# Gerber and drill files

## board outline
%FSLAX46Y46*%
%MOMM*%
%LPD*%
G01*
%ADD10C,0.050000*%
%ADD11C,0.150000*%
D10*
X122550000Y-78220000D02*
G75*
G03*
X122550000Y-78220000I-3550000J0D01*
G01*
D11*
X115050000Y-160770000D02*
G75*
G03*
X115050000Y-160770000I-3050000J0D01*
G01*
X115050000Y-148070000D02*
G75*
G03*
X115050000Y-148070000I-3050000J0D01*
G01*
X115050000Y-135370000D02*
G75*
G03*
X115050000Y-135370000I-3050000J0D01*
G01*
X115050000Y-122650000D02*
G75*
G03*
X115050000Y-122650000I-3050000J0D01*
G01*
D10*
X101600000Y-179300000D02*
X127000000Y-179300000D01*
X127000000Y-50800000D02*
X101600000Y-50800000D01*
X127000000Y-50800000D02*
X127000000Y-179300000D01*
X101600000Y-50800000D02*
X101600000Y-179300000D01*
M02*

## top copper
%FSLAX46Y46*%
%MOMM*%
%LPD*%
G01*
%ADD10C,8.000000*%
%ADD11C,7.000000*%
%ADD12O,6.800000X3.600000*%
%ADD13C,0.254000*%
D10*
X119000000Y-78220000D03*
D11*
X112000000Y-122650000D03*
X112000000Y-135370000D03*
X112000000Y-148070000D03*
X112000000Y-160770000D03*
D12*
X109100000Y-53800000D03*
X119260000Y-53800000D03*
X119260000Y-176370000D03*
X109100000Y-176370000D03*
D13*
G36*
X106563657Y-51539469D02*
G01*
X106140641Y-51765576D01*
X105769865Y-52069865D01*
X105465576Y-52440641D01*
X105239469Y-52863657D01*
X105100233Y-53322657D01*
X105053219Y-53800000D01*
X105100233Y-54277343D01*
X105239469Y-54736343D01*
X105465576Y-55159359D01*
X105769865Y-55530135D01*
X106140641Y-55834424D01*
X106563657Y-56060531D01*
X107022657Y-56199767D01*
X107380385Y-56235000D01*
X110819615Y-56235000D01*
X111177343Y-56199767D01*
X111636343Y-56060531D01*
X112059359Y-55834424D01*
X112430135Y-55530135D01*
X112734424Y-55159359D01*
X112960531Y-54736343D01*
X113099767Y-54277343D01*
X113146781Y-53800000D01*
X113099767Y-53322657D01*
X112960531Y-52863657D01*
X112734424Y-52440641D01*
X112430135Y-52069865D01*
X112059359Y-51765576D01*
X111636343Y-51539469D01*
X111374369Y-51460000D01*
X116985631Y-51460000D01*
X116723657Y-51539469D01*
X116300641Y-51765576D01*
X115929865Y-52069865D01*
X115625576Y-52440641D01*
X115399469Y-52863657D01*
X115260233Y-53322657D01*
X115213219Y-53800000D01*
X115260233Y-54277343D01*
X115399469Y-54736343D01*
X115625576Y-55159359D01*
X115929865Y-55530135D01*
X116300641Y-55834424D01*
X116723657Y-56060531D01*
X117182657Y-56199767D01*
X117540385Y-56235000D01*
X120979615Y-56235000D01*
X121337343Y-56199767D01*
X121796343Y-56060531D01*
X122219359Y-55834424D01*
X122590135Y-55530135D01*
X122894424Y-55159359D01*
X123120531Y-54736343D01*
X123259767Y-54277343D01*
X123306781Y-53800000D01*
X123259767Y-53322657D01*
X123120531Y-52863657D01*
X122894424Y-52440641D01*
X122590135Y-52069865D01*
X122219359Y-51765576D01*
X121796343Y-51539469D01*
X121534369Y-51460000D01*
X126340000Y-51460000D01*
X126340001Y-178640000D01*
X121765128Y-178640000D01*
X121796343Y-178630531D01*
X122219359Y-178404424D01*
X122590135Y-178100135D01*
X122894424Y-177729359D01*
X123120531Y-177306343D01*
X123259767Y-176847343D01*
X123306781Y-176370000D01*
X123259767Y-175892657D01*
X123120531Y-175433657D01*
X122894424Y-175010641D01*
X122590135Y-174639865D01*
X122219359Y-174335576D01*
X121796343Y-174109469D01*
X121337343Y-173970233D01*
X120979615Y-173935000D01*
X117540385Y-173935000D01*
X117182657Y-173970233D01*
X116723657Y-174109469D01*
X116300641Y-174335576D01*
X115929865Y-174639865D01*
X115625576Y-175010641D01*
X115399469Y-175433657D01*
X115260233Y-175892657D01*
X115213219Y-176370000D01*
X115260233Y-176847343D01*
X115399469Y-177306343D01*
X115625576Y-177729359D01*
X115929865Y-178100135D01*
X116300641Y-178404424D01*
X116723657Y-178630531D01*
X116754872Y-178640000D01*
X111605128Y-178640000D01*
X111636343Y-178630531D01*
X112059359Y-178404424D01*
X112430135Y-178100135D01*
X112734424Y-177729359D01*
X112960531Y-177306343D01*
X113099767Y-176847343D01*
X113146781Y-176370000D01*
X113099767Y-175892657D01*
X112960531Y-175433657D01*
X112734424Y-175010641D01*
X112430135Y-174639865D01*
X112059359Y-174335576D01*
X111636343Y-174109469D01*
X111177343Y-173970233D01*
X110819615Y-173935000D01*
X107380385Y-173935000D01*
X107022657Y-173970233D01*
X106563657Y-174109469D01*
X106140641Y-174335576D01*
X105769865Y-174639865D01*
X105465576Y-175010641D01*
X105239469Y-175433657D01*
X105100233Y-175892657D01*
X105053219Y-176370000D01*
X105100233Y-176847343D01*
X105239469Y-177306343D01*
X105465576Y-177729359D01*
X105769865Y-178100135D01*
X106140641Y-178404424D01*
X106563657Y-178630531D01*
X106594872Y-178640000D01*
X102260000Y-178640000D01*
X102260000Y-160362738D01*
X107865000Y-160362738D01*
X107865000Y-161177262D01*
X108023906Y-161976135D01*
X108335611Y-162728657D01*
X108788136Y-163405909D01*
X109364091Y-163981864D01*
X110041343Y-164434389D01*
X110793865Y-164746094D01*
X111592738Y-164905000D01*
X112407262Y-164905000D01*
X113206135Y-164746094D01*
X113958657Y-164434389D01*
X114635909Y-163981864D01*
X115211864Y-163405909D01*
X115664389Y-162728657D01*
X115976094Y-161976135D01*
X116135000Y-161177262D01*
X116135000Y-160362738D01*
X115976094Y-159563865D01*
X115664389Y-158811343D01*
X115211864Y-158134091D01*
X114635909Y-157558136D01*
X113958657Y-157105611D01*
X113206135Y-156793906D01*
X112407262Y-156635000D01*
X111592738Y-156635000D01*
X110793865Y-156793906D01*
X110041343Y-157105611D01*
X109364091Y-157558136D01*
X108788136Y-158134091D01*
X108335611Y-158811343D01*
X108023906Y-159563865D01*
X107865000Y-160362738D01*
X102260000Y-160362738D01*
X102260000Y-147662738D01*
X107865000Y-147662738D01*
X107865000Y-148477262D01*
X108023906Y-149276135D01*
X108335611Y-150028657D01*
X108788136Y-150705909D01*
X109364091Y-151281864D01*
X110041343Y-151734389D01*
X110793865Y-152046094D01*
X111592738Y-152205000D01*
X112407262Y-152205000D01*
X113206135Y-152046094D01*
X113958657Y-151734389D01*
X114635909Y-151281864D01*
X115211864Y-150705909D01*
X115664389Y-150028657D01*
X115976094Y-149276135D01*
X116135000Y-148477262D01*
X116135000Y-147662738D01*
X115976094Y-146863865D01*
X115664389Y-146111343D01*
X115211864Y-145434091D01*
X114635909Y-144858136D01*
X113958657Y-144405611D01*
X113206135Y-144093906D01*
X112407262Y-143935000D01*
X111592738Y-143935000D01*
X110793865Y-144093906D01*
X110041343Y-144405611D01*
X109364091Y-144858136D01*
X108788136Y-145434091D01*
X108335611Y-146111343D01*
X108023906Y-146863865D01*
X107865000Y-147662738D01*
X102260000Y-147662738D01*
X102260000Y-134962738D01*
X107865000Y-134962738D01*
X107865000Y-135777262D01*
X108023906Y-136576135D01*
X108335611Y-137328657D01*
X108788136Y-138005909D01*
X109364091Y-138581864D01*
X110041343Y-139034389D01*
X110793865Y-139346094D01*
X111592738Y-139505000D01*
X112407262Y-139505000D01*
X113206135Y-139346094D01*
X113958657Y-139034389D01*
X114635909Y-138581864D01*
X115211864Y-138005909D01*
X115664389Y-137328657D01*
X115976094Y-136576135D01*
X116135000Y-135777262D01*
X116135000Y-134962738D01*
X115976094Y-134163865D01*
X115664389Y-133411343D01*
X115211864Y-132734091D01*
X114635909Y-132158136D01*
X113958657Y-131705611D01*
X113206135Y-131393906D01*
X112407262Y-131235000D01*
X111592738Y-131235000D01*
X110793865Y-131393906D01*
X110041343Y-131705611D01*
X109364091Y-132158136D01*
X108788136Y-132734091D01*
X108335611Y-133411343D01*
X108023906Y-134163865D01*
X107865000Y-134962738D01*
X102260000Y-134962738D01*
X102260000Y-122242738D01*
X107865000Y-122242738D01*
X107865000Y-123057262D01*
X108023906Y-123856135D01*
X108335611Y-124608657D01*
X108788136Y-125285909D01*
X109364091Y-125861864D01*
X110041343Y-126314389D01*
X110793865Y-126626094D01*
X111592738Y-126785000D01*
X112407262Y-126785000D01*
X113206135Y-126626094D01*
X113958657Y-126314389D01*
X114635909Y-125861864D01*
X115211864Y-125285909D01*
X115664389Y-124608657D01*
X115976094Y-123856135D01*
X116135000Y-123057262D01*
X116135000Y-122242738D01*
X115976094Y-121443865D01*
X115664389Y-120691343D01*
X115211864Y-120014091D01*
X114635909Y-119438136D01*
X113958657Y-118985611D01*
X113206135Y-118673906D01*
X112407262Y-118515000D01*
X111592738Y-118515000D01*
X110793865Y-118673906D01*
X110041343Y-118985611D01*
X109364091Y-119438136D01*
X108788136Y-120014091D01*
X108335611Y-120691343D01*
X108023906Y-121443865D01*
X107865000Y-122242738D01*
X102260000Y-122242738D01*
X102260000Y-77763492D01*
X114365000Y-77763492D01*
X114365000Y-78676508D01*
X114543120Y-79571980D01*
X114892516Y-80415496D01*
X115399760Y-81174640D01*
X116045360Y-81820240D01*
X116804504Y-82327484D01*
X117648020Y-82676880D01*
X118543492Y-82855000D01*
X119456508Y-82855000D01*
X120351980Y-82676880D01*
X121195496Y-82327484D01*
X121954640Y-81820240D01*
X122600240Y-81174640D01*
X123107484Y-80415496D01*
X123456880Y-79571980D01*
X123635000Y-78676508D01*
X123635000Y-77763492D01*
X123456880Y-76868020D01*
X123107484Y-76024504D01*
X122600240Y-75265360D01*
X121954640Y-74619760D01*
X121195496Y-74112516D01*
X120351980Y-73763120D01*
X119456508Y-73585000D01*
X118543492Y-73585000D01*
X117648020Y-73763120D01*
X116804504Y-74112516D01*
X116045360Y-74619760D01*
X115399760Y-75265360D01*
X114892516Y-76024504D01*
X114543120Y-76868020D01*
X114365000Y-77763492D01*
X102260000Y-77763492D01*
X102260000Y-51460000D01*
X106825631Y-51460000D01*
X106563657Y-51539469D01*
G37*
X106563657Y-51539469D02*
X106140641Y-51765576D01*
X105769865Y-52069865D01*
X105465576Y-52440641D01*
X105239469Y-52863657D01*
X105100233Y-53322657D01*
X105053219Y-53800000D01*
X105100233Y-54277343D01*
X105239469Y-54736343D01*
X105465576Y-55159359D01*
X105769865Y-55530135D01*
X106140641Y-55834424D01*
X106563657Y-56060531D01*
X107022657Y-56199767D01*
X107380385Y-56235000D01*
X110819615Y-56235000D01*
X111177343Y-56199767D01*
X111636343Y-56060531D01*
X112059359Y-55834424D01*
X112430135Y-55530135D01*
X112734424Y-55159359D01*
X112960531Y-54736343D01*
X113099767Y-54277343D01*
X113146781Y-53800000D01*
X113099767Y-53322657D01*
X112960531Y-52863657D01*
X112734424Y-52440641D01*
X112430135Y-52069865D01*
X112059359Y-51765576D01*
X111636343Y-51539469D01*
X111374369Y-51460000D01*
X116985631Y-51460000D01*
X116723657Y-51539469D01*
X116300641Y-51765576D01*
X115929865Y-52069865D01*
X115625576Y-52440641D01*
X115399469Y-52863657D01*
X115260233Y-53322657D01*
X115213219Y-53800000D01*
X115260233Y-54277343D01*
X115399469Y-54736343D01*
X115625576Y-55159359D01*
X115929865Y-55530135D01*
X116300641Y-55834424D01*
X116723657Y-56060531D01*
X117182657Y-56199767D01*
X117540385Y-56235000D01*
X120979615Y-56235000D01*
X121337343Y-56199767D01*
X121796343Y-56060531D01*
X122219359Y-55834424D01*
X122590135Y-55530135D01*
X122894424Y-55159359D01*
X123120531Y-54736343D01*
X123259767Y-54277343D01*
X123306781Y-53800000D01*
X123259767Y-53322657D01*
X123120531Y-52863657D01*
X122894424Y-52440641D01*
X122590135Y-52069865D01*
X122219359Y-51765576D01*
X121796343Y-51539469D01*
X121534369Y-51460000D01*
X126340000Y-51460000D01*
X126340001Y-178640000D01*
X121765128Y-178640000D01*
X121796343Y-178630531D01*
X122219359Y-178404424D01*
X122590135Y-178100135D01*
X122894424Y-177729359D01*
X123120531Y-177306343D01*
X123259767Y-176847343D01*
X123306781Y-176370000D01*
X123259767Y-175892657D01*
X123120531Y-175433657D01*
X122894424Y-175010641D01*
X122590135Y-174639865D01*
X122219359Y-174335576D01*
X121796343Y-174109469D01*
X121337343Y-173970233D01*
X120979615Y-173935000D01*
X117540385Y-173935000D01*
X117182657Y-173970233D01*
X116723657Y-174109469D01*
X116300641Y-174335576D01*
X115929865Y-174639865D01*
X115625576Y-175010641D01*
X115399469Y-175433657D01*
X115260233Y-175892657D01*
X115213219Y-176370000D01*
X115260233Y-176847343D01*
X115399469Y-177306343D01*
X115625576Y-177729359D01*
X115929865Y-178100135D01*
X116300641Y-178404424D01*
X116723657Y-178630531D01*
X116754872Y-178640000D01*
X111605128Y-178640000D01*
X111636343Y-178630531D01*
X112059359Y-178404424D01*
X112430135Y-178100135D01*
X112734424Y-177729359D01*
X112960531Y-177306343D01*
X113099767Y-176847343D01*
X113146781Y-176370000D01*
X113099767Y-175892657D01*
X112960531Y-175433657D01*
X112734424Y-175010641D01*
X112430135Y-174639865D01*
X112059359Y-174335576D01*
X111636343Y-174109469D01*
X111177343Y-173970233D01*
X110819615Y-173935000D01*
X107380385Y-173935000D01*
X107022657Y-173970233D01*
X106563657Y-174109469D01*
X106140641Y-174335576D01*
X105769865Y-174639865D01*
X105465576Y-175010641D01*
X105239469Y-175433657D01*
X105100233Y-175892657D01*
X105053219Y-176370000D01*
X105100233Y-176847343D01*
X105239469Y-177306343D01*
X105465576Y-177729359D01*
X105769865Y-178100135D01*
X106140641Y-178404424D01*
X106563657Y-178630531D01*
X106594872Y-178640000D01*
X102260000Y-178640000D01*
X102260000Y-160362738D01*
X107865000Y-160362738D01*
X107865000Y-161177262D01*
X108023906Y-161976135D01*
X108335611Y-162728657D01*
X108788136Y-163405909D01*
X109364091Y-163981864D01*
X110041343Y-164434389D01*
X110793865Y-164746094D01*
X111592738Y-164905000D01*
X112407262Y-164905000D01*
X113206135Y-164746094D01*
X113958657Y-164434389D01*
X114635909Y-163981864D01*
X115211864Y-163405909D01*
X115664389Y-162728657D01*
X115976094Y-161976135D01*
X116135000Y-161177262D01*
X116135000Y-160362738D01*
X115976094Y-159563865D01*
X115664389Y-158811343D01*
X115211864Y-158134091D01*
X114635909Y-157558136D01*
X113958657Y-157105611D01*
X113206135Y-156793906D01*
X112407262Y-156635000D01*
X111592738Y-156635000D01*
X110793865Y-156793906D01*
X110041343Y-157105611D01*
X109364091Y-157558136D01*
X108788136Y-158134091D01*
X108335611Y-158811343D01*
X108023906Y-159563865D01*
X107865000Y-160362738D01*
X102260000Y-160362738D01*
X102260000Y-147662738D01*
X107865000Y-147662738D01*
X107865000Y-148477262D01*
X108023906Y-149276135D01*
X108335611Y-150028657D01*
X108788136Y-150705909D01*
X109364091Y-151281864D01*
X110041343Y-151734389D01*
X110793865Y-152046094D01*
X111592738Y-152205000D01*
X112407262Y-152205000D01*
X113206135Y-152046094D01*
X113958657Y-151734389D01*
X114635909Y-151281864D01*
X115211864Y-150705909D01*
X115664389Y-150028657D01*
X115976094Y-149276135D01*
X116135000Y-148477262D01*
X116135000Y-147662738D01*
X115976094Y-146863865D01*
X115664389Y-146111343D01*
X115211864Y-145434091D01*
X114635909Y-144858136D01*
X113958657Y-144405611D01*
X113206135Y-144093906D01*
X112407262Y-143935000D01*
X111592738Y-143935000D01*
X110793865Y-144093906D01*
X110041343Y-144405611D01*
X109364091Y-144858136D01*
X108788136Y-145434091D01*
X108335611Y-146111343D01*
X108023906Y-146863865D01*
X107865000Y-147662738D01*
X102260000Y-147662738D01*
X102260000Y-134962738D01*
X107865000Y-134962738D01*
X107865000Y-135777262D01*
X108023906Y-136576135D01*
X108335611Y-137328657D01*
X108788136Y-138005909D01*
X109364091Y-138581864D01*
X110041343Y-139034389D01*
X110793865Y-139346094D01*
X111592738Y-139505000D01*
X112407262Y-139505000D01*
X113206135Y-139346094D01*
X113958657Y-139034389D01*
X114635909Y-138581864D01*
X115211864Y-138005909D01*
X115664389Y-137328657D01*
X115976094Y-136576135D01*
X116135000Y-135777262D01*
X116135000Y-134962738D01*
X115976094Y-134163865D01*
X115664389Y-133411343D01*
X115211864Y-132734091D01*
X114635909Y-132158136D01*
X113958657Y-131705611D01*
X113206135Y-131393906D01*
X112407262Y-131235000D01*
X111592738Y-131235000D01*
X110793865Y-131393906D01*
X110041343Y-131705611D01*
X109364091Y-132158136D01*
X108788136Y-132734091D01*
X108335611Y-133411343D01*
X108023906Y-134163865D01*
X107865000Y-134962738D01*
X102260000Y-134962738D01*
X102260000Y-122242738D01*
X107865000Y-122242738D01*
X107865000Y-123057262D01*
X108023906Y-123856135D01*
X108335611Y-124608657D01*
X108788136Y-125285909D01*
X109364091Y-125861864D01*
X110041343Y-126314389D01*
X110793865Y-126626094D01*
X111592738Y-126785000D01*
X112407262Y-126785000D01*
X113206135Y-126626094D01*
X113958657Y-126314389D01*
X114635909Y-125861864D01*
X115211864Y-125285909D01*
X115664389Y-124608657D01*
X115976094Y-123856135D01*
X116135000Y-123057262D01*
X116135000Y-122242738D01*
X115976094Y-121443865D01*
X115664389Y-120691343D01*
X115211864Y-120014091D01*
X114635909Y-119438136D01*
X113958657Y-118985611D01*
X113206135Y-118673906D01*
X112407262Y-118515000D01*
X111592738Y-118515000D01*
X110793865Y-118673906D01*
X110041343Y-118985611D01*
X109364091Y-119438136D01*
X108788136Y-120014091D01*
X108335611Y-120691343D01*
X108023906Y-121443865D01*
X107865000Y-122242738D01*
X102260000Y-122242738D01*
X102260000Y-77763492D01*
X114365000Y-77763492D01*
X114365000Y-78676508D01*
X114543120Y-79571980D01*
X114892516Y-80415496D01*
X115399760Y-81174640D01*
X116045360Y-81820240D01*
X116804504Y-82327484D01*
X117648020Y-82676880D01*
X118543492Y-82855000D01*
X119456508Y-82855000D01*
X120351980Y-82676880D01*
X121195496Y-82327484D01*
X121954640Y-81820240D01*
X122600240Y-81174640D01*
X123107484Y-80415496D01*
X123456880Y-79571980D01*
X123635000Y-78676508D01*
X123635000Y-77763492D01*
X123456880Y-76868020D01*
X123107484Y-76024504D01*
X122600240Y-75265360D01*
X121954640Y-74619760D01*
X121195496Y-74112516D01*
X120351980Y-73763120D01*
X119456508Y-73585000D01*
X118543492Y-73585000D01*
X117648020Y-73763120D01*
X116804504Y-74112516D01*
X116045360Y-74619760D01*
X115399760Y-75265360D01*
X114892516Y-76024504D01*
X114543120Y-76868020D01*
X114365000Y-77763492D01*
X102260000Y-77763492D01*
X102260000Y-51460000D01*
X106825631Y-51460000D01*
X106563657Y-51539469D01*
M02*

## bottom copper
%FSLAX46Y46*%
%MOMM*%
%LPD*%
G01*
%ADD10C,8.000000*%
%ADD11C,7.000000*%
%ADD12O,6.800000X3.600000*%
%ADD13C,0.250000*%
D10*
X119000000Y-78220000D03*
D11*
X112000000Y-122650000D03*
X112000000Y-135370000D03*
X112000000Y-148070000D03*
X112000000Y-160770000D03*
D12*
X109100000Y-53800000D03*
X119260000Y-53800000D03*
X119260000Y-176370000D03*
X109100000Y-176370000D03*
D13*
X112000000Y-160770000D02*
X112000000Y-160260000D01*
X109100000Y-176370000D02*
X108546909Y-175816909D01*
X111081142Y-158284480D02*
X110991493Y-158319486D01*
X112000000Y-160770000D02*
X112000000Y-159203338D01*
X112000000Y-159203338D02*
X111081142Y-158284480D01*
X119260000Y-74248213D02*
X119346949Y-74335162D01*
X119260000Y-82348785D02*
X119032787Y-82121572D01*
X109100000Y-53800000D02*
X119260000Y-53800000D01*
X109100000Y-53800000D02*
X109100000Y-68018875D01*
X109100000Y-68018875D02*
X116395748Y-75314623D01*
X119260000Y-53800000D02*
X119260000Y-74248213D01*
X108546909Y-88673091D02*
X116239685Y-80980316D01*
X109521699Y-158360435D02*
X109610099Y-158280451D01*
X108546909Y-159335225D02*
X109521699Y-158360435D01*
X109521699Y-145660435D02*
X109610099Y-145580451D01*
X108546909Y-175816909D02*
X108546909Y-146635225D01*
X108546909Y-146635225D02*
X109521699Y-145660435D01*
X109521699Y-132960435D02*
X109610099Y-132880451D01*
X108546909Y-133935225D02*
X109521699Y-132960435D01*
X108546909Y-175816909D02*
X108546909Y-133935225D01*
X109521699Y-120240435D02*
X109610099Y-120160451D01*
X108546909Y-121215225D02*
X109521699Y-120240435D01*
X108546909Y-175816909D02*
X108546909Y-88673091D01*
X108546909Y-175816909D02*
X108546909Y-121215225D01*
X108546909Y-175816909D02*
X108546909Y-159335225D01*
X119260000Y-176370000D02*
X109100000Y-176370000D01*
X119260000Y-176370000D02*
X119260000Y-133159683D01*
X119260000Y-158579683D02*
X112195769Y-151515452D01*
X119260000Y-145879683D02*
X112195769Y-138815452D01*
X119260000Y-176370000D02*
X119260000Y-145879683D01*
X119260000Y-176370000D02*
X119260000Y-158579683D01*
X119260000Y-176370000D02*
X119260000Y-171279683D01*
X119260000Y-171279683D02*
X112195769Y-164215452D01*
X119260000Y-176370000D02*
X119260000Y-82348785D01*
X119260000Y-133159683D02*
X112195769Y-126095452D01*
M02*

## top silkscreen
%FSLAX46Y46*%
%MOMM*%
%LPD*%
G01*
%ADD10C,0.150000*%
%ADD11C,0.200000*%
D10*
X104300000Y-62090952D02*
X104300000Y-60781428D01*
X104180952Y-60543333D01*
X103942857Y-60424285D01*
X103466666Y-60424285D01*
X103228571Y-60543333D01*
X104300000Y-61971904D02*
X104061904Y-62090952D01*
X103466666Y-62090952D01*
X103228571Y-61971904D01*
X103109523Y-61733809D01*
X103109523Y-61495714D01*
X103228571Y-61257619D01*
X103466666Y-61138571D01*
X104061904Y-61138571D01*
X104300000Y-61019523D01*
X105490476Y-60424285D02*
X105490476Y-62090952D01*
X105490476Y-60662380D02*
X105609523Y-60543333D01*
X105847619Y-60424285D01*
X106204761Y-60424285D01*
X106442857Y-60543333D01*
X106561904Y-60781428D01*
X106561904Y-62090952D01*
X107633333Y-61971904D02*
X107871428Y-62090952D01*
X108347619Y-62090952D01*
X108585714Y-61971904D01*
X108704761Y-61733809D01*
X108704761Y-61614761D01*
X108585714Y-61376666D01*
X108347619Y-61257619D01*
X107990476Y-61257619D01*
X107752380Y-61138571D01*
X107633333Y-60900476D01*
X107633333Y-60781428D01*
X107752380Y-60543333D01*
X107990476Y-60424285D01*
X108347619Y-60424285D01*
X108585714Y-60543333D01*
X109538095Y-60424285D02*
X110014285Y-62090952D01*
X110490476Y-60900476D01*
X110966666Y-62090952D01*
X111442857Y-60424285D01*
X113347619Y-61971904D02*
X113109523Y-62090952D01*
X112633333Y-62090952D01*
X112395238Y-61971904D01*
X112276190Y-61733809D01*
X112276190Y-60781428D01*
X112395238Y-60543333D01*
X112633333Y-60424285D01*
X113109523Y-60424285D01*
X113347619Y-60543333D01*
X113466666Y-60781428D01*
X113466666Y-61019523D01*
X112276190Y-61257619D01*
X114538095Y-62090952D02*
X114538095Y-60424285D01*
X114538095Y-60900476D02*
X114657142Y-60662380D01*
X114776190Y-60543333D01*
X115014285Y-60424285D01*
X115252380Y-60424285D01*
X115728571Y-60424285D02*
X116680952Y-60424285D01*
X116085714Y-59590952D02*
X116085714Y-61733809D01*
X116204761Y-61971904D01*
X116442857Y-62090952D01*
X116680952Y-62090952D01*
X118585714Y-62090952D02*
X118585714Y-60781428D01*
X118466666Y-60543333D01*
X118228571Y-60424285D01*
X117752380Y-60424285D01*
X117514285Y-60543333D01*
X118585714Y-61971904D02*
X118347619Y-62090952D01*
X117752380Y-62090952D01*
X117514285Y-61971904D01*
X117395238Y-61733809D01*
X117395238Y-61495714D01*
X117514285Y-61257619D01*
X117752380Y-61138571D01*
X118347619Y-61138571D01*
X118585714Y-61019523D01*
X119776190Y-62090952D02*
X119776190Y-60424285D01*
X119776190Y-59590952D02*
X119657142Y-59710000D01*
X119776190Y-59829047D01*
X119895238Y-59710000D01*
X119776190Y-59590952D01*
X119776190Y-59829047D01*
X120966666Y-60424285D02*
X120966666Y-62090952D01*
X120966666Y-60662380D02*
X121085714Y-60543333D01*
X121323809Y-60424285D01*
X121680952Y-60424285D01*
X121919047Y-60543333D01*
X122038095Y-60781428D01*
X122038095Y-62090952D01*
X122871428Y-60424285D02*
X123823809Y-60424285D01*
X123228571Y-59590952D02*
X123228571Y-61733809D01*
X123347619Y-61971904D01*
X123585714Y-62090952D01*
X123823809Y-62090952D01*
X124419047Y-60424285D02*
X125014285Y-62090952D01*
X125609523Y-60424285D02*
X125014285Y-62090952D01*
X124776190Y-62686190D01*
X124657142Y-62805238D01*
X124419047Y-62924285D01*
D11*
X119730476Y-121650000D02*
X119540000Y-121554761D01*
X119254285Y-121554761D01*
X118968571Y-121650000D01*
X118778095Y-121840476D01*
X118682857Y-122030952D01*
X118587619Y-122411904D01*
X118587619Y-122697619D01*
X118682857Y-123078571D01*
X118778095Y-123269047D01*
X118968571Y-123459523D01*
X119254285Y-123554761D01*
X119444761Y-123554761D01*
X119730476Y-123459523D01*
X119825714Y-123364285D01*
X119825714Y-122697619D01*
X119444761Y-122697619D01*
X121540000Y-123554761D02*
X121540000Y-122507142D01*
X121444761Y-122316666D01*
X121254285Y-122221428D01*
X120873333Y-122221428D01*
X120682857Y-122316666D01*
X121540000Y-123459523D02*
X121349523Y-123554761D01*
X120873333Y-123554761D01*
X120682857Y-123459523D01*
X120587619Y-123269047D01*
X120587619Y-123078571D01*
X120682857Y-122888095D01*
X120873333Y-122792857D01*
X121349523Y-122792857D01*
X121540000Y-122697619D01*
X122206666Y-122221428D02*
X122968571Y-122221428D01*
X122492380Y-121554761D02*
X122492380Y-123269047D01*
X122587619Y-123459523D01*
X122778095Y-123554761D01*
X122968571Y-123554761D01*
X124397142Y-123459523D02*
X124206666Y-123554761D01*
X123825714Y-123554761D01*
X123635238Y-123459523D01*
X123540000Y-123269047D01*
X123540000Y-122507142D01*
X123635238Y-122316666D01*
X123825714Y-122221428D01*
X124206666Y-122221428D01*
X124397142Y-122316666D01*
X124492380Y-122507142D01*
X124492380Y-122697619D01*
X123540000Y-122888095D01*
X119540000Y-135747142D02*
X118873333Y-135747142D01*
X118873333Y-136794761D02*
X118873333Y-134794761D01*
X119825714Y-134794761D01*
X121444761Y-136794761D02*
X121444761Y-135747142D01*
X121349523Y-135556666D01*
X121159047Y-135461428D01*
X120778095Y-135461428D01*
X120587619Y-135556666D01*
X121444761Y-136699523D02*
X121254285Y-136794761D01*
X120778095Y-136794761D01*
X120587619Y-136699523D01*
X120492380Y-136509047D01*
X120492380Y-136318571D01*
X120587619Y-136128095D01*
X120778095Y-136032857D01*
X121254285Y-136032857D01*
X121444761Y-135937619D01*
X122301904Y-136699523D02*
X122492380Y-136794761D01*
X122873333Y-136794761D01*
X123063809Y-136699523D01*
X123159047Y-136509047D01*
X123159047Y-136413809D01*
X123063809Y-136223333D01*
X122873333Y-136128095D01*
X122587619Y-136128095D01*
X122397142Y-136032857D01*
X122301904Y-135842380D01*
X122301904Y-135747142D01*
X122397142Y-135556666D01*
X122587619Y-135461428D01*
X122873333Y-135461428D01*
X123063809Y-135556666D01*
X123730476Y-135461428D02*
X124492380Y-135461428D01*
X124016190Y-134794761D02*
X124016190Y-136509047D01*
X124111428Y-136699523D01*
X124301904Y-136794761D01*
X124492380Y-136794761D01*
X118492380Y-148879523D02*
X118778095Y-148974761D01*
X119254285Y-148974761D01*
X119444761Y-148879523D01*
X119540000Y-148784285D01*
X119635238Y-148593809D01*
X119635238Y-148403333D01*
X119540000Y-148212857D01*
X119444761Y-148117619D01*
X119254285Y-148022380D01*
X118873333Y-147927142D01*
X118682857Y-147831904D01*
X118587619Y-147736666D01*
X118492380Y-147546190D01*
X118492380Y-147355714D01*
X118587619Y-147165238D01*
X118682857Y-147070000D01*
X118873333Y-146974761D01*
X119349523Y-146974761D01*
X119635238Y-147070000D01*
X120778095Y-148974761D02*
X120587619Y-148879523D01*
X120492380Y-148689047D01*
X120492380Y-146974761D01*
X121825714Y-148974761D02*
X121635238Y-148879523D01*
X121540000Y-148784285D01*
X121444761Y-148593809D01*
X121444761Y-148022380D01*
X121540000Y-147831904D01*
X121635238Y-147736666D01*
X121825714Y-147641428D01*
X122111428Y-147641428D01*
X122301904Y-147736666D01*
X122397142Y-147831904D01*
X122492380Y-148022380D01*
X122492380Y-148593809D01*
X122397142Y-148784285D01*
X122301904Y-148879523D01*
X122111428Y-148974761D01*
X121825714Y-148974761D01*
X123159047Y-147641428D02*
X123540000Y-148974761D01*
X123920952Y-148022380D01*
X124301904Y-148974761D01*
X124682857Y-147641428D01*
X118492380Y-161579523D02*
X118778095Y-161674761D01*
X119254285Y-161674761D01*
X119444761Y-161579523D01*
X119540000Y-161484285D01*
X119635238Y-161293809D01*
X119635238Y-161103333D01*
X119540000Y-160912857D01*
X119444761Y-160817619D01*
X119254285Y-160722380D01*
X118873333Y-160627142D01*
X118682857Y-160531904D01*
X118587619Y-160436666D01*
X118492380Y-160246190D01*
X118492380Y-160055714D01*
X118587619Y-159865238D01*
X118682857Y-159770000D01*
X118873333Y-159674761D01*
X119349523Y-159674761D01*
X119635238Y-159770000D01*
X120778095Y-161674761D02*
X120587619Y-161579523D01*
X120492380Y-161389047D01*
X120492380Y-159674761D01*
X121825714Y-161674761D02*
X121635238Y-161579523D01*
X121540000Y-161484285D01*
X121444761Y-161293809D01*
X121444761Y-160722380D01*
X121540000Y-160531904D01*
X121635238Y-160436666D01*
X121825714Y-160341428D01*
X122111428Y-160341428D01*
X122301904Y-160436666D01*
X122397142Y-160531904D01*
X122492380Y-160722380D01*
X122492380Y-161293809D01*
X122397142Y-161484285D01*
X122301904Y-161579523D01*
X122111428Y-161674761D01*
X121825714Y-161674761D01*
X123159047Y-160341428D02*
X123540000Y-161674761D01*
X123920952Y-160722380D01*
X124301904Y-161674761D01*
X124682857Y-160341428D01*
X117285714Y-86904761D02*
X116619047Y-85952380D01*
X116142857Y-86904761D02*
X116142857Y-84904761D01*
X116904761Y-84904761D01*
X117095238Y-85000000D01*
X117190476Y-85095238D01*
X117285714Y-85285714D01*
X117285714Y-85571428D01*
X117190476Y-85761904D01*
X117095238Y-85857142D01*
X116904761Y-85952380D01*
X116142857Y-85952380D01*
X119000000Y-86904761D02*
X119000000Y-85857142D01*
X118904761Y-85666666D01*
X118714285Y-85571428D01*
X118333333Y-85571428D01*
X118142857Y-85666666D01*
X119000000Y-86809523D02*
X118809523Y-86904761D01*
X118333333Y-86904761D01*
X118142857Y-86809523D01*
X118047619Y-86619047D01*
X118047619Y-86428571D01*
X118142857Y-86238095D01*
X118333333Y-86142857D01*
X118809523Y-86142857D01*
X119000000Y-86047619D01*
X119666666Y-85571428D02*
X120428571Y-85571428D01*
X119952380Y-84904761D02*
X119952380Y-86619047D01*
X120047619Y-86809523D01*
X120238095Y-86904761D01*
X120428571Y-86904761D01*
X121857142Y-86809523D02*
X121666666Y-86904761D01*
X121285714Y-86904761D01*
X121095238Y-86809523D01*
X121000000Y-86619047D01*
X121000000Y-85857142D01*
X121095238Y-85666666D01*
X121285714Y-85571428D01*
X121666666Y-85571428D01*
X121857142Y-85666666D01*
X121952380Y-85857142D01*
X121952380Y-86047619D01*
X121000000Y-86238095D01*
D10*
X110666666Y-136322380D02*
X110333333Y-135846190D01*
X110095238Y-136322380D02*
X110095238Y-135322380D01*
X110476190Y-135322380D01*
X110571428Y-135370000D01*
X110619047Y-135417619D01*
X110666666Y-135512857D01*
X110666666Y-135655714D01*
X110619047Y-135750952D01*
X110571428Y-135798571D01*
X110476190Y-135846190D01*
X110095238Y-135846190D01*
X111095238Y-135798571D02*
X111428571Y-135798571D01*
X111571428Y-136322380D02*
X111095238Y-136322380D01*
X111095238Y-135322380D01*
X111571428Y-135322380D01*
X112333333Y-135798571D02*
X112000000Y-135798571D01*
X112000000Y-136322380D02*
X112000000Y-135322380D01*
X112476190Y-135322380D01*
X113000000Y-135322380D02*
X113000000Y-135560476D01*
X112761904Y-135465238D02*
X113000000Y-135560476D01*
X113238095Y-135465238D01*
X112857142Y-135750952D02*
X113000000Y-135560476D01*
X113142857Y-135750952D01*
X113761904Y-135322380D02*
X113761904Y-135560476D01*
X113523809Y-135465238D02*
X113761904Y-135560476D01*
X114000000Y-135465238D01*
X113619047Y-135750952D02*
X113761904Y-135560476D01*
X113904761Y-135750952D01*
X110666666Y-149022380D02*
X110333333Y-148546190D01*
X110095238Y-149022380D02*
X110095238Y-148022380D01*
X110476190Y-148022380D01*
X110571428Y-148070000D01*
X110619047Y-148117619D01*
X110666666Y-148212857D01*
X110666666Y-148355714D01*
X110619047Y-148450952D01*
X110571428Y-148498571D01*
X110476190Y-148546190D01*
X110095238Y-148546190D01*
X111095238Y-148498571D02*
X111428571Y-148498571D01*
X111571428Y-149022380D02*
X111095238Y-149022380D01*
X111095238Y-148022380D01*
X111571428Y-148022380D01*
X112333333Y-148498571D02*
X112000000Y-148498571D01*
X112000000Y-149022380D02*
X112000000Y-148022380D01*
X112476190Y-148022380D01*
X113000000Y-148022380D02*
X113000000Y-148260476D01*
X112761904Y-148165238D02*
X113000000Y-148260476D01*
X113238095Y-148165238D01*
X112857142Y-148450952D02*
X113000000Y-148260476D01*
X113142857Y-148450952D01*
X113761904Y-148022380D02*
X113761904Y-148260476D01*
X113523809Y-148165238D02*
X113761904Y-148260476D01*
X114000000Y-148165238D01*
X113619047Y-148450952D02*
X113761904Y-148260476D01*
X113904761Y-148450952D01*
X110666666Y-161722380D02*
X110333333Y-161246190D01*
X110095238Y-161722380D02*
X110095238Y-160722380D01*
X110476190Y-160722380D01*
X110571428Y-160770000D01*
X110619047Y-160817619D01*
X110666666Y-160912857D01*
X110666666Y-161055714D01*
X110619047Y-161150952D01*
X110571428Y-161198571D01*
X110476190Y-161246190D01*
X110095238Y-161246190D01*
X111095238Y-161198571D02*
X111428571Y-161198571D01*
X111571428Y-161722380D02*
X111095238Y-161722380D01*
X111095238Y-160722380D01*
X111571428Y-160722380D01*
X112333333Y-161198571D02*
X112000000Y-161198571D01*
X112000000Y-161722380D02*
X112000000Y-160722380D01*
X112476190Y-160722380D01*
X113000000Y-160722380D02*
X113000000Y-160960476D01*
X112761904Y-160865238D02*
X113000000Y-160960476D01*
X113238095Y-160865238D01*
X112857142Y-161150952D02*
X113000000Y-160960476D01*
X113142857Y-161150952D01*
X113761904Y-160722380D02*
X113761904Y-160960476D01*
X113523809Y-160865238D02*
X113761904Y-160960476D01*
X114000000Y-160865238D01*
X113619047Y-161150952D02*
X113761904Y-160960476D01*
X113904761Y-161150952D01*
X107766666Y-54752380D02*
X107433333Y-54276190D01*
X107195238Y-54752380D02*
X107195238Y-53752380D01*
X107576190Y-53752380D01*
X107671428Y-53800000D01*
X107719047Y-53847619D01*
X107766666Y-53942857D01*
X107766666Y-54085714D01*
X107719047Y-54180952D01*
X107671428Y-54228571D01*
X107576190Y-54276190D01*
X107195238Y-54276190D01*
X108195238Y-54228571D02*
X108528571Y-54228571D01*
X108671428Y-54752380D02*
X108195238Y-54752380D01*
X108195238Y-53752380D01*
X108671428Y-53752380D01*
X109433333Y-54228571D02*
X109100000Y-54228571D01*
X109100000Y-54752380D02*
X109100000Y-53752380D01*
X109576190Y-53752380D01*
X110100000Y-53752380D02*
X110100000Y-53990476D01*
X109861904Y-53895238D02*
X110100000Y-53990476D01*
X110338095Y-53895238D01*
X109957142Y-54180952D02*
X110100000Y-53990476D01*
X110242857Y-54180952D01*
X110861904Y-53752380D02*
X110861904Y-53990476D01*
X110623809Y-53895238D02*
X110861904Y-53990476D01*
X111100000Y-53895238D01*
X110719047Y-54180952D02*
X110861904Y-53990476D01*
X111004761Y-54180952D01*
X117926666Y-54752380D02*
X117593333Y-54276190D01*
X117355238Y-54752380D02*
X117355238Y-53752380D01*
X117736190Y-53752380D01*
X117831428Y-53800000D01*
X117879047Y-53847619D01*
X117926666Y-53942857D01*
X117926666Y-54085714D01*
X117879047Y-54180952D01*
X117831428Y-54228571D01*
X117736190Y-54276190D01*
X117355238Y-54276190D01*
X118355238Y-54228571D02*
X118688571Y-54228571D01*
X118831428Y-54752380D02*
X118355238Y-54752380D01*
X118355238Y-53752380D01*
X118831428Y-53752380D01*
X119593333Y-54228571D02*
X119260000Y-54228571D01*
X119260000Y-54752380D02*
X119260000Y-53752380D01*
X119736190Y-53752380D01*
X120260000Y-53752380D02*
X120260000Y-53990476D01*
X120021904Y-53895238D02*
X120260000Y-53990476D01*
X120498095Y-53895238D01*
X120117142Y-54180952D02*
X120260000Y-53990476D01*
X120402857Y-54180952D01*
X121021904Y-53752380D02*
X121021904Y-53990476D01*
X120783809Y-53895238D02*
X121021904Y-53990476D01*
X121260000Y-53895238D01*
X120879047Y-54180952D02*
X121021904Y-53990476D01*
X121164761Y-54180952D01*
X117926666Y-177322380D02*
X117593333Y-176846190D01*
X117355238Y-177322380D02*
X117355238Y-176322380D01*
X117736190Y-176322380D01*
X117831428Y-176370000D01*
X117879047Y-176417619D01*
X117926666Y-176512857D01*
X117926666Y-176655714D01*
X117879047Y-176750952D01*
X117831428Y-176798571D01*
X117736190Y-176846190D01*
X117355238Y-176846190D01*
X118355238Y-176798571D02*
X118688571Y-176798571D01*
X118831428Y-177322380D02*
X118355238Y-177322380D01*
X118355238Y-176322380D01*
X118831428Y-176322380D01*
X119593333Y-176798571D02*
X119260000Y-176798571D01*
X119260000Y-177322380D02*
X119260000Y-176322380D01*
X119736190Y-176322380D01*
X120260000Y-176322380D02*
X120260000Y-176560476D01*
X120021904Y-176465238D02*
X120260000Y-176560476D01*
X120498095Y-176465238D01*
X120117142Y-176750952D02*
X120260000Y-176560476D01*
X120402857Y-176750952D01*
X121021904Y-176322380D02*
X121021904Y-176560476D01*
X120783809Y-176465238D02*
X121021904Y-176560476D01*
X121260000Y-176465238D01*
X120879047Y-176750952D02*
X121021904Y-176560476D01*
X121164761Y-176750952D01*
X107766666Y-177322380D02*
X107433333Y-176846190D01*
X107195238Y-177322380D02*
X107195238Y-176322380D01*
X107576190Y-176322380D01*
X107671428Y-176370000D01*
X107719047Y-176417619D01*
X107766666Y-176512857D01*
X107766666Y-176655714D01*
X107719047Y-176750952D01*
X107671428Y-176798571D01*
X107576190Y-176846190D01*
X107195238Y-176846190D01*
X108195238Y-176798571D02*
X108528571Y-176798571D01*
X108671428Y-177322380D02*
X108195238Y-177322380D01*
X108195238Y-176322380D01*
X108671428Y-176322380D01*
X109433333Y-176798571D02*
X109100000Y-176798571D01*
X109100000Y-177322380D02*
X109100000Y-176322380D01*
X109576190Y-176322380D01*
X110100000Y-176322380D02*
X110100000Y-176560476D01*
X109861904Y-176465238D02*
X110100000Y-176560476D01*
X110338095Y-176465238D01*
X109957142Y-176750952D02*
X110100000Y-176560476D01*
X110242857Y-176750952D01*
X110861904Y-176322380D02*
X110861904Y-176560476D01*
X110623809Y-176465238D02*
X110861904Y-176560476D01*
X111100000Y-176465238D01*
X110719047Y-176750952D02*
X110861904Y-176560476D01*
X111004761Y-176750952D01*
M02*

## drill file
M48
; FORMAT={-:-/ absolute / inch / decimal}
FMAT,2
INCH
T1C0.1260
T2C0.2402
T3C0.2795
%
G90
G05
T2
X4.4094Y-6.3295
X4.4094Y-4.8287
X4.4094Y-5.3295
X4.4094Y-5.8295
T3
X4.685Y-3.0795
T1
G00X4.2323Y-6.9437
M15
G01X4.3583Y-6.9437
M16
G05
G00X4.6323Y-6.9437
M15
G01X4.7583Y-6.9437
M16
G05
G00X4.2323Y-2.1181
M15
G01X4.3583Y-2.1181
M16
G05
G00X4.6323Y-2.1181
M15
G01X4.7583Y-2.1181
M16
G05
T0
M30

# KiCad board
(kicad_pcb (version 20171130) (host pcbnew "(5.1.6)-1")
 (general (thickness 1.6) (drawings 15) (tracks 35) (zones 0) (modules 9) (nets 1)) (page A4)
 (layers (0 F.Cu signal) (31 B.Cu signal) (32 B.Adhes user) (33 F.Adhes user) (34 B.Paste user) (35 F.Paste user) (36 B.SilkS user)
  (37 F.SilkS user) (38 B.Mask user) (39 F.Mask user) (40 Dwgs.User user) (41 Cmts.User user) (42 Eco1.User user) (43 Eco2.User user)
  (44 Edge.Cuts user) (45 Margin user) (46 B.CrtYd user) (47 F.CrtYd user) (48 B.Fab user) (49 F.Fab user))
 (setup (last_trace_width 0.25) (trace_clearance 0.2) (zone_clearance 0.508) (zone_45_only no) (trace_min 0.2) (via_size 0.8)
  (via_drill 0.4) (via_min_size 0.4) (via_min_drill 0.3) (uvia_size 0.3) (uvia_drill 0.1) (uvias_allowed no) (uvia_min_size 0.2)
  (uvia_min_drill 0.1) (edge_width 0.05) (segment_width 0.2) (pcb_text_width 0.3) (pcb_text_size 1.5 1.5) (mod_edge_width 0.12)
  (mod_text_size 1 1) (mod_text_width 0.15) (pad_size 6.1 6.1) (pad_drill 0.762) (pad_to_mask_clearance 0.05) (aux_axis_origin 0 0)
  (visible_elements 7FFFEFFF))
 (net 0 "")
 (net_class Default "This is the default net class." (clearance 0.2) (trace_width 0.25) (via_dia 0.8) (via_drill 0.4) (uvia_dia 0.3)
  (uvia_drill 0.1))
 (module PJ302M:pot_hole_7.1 (layer F.Cu) (at 119 78.22)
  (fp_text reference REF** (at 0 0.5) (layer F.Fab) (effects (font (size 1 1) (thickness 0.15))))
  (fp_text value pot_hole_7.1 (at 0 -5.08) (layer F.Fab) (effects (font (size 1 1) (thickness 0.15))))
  (pad "" np_thru_hole circle (at 0 0) (size 8 8) (drill 7.1) (layers *.Cu *.Mask)))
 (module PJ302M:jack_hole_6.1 (layer F.Cu) (at 112 122.65)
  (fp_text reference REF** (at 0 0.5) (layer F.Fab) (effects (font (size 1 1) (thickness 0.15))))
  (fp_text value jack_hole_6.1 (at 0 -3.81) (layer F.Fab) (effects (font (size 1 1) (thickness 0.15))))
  (pad "" np_thru_hole circle (at 0 0 90) (size 7 7) (drill 6.1) (layers *.Cu *.Mask)))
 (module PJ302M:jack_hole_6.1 (layer F.Cu) (at 112 135.37)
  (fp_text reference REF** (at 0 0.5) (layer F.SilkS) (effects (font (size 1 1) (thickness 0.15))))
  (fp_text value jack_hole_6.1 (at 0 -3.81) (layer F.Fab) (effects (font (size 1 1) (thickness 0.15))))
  (pad "" np_thru_hole circle (at 0 0 90) (size 7 7) (drill 6.1) (layers *.Cu *.Mask)))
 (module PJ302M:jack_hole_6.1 (layer F.Cu) (at 112 148.07)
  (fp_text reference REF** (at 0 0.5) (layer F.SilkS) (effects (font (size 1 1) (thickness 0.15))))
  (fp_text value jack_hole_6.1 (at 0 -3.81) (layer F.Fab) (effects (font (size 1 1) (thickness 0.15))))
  (pad "" np_thru_hole circle (at 0 0 90) (size 7 7) (drill 6.1) (layers *.Cu *.Mask)))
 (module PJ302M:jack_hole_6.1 (layer F.Cu) (at 112 160.77)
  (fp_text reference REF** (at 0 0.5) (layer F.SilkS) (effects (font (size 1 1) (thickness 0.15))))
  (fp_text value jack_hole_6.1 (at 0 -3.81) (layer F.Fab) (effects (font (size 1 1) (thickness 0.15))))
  (pad "" np_thru_hole circle (at 0 0 90) (size 7 7) (drill 6.1) (layers *.Cu *.Mask)))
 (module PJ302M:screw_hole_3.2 (layer F.Cu) (at 109.1 53.8)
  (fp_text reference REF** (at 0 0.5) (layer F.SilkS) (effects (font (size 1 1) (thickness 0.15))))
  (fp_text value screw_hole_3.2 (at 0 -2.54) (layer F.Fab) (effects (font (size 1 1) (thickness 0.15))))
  (pad "" np_thru_hole oval (at 0 0 90) (size 3.6 6.8) (drill oval 3.2 6.4) (layers *.Cu *.Mask)))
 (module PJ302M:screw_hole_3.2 (layer F.Cu) (at 119.26 53.8)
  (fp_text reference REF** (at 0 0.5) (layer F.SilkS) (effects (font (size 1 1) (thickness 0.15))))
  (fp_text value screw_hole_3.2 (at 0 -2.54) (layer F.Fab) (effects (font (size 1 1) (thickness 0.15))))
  (pad "" np_thru_hole oval (at 0 0 90) (size 3.6 6.8) (drill oval 3.2 6.4) (layers *.Cu *.Mask)))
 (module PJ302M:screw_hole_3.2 (layer F.Cu) (at 119.26 176.37)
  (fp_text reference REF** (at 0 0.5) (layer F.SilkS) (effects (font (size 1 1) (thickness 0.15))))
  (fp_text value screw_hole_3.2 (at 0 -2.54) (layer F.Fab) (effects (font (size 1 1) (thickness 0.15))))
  (pad "" np_thru_hole oval (at 0 0 90) (size 3.6 6.8) (drill oval 3.2 6.4) (layers *.Cu *.Mask)))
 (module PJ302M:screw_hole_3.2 (layer F.Cu) (at 109.1 176.37)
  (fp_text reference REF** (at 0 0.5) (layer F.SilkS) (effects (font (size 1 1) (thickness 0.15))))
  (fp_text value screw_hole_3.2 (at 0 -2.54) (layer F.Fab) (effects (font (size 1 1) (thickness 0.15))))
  (pad "" np_thru_hole oval (at 0 0 90) (size 3.6 6.8) (drill oval 3.2 6.4) (layers *.Cu *.Mask)))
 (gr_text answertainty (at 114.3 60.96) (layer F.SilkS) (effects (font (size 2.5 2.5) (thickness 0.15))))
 (gr_circle (center 119 78.22) (end 122.55 78.22) (layer Edge.Cuts) (width 0.05))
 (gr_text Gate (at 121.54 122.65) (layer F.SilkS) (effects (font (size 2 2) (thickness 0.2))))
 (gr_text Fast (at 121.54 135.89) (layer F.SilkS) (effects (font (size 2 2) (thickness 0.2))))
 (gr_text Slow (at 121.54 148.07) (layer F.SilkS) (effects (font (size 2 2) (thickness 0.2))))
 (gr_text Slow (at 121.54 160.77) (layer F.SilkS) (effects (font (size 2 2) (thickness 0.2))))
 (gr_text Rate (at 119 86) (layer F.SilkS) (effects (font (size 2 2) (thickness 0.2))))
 (gr_circle (center 112 160.77) (end 115.05 160.77) (layer Edge.Cuts) (width 0.15))
 (gr_circle (center 112 148.07) (end 115.05 148.07) (layer Edge.Cuts) (width 0.15))
 (gr_circle (center 112 135.37) (end 115.05 135.37) (layer Edge.Cuts) (width 0.15))
 (gr_circle (center 112 122.65) (end 115.05 122.65) (layer Edge.Cuts) (width 0.15))
 (gr_line (start 101.6 179.3) (end 127 179.3) (layer Edge.Cuts) (width 0.05))
 (gr_line (start 127 50.8) (end 101.6 50.8) (layer Edge.Cuts) (width 0.05))
 (gr_line (start 127 50.8) (end 127 179.3) (layer Edge.Cuts) (width 0.05))
 (gr_line (start 101.6 50.8) (end 101.6 179.3) (layer Edge.Cuts) (width 0.05))
 (segment (start 112 160.77) (end 112 160.26) (width 0.25) (layer B.Cu) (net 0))
 (segment (start 109.1 176.37) (end 108.546909 175.816909) (width 0.25) (layer B.Cu) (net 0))
 (segment (start 111.081142 158.28448) (end 110.991493 158.319486) (width 0.25) (layer B.Cu) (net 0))
 (segment (start 112 160.77) (end 112 159.203338) (width 0.25) (layer B.Cu) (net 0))
 (segment (start 112 159.203338) (end 111.081142 158.28448) (width 0.25) (layer B.Cu) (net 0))
 (segment (start 119.26 74.248213) (end 119.346949 74.335162) (width 0.25) (layer B.Cu) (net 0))
 (segment (start 119.26 82.348785) (end 119.032787 82.121572) (width 0.25) (layer B.Cu) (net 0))
 (segment (start 109.1 53.8) (end 119.26 53.8) (width 0.25) (layer B.Cu) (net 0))
 (segment (start 109.1 53.8) (end 109.1 68.018875) (width 0.25) (layer B.Cu) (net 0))
 (segment (start 109.1 68.018875) (end 116.395748 75.314623) (width 0.25) (layer B.Cu) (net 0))
 (segment (start 119.26 53.8) (end 119.26 74.248213) (width 0.25) (layer B.Cu) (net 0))
 (segment (start 108.546909 88.673091) (end 116.239685 80.980316) (width 0.25) (layer B.Cu) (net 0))
 (segment (start 109.521699 158.360435) (end 109.610099 158.280451) (width 0.25) (layer B.Cu) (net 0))
 (segment (start 108.546909 159.335225) (end 109.521699 158.360435) (width 0.25) (layer B.Cu) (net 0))
 (segment (start 109.521699 145.660435) (end 109.610099 145.580451) (width 0.25) (layer B.Cu) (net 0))
 (segment (start 108.546909 175.816909) (end 108.546909 146.635225) (width 0.25) (layer B.Cu) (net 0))
 (segment (start 108.546909 146.635225) (end 109.521699 145.660435) (width 0.25) (layer B.Cu) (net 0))
 (segment (start 109.521699 132.960435) (end 109.610099 132.880451) (width 0.25) (layer B.Cu) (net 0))
 (segment (start 108.546909 133.935225) (end 109.521699 132.960435) (width 0.25) (layer B.Cu) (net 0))
 (segment (start 108.546909 175.816909) (end 108.546909 133.935225) (width 0.25) (layer B.Cu) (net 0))
 (segment (start 109.521699 120.240435) (end 109.610099 120.160451) (width 0.25) (layer B.Cu) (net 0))
 (segment (start 108.546909 121.215225) (end 109.521699 120.240435) (width 0.25) (layer B.Cu) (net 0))
 (segment (start 108.546909 175.816909) (end 108.546909 88.673091) (width 0.25) (layer B.Cu) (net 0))
 (segment (start 108.546909 175.816909) (end 108.546909 121.215225) (width 0.25) (layer B.Cu) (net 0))
 (segment (start 108.546909 175.816909) (end 108.546909 159.335225) (width 0.25) (layer B.Cu) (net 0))
 (segment (start 119.26 176.37) (end 109.1 176.37) (width 0.25) (layer B.Cu) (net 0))
 (segment (start 119.26 176.37) (end 119.26 133.159683) (width 0.25) (layer B.Cu) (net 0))
 (segment (start 119.26 158.579683) (end 112.195769 151.515452) (width 0.25) (layer B.Cu) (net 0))
 (segment (start 119.26 145.879683) (end 112.195769 138.815452) (width 0.25) (layer B.Cu) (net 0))
 (segment (start 119.26 176.37) (end 119.26 145.879683) (width 0.25) (layer B.Cu) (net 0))
 (segment (start 119.26 176.37) (end 119.26 158.579683) (width 0.25) (layer B.Cu) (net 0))
 (segment (start 119.26 176.37) (end 119.26 171.279683) (width 0.25) (layer B.Cu) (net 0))
 (segment (start 119.26 171.279683) (end 112.195769 164.215452) (width 0.25) (layer B.Cu) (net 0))
 (segment (start 119.26 176.37) (end 119.26 82.348785) (width 0.25) (layer B.Cu) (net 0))
 (segment (start 119.26 133.159683) (end 112.195769 126.095452) (width 0.25) (layer B.Cu) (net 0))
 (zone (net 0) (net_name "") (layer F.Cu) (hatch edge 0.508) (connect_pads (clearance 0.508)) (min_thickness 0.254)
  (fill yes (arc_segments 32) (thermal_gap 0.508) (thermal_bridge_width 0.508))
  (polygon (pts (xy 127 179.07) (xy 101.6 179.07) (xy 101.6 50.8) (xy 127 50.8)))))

